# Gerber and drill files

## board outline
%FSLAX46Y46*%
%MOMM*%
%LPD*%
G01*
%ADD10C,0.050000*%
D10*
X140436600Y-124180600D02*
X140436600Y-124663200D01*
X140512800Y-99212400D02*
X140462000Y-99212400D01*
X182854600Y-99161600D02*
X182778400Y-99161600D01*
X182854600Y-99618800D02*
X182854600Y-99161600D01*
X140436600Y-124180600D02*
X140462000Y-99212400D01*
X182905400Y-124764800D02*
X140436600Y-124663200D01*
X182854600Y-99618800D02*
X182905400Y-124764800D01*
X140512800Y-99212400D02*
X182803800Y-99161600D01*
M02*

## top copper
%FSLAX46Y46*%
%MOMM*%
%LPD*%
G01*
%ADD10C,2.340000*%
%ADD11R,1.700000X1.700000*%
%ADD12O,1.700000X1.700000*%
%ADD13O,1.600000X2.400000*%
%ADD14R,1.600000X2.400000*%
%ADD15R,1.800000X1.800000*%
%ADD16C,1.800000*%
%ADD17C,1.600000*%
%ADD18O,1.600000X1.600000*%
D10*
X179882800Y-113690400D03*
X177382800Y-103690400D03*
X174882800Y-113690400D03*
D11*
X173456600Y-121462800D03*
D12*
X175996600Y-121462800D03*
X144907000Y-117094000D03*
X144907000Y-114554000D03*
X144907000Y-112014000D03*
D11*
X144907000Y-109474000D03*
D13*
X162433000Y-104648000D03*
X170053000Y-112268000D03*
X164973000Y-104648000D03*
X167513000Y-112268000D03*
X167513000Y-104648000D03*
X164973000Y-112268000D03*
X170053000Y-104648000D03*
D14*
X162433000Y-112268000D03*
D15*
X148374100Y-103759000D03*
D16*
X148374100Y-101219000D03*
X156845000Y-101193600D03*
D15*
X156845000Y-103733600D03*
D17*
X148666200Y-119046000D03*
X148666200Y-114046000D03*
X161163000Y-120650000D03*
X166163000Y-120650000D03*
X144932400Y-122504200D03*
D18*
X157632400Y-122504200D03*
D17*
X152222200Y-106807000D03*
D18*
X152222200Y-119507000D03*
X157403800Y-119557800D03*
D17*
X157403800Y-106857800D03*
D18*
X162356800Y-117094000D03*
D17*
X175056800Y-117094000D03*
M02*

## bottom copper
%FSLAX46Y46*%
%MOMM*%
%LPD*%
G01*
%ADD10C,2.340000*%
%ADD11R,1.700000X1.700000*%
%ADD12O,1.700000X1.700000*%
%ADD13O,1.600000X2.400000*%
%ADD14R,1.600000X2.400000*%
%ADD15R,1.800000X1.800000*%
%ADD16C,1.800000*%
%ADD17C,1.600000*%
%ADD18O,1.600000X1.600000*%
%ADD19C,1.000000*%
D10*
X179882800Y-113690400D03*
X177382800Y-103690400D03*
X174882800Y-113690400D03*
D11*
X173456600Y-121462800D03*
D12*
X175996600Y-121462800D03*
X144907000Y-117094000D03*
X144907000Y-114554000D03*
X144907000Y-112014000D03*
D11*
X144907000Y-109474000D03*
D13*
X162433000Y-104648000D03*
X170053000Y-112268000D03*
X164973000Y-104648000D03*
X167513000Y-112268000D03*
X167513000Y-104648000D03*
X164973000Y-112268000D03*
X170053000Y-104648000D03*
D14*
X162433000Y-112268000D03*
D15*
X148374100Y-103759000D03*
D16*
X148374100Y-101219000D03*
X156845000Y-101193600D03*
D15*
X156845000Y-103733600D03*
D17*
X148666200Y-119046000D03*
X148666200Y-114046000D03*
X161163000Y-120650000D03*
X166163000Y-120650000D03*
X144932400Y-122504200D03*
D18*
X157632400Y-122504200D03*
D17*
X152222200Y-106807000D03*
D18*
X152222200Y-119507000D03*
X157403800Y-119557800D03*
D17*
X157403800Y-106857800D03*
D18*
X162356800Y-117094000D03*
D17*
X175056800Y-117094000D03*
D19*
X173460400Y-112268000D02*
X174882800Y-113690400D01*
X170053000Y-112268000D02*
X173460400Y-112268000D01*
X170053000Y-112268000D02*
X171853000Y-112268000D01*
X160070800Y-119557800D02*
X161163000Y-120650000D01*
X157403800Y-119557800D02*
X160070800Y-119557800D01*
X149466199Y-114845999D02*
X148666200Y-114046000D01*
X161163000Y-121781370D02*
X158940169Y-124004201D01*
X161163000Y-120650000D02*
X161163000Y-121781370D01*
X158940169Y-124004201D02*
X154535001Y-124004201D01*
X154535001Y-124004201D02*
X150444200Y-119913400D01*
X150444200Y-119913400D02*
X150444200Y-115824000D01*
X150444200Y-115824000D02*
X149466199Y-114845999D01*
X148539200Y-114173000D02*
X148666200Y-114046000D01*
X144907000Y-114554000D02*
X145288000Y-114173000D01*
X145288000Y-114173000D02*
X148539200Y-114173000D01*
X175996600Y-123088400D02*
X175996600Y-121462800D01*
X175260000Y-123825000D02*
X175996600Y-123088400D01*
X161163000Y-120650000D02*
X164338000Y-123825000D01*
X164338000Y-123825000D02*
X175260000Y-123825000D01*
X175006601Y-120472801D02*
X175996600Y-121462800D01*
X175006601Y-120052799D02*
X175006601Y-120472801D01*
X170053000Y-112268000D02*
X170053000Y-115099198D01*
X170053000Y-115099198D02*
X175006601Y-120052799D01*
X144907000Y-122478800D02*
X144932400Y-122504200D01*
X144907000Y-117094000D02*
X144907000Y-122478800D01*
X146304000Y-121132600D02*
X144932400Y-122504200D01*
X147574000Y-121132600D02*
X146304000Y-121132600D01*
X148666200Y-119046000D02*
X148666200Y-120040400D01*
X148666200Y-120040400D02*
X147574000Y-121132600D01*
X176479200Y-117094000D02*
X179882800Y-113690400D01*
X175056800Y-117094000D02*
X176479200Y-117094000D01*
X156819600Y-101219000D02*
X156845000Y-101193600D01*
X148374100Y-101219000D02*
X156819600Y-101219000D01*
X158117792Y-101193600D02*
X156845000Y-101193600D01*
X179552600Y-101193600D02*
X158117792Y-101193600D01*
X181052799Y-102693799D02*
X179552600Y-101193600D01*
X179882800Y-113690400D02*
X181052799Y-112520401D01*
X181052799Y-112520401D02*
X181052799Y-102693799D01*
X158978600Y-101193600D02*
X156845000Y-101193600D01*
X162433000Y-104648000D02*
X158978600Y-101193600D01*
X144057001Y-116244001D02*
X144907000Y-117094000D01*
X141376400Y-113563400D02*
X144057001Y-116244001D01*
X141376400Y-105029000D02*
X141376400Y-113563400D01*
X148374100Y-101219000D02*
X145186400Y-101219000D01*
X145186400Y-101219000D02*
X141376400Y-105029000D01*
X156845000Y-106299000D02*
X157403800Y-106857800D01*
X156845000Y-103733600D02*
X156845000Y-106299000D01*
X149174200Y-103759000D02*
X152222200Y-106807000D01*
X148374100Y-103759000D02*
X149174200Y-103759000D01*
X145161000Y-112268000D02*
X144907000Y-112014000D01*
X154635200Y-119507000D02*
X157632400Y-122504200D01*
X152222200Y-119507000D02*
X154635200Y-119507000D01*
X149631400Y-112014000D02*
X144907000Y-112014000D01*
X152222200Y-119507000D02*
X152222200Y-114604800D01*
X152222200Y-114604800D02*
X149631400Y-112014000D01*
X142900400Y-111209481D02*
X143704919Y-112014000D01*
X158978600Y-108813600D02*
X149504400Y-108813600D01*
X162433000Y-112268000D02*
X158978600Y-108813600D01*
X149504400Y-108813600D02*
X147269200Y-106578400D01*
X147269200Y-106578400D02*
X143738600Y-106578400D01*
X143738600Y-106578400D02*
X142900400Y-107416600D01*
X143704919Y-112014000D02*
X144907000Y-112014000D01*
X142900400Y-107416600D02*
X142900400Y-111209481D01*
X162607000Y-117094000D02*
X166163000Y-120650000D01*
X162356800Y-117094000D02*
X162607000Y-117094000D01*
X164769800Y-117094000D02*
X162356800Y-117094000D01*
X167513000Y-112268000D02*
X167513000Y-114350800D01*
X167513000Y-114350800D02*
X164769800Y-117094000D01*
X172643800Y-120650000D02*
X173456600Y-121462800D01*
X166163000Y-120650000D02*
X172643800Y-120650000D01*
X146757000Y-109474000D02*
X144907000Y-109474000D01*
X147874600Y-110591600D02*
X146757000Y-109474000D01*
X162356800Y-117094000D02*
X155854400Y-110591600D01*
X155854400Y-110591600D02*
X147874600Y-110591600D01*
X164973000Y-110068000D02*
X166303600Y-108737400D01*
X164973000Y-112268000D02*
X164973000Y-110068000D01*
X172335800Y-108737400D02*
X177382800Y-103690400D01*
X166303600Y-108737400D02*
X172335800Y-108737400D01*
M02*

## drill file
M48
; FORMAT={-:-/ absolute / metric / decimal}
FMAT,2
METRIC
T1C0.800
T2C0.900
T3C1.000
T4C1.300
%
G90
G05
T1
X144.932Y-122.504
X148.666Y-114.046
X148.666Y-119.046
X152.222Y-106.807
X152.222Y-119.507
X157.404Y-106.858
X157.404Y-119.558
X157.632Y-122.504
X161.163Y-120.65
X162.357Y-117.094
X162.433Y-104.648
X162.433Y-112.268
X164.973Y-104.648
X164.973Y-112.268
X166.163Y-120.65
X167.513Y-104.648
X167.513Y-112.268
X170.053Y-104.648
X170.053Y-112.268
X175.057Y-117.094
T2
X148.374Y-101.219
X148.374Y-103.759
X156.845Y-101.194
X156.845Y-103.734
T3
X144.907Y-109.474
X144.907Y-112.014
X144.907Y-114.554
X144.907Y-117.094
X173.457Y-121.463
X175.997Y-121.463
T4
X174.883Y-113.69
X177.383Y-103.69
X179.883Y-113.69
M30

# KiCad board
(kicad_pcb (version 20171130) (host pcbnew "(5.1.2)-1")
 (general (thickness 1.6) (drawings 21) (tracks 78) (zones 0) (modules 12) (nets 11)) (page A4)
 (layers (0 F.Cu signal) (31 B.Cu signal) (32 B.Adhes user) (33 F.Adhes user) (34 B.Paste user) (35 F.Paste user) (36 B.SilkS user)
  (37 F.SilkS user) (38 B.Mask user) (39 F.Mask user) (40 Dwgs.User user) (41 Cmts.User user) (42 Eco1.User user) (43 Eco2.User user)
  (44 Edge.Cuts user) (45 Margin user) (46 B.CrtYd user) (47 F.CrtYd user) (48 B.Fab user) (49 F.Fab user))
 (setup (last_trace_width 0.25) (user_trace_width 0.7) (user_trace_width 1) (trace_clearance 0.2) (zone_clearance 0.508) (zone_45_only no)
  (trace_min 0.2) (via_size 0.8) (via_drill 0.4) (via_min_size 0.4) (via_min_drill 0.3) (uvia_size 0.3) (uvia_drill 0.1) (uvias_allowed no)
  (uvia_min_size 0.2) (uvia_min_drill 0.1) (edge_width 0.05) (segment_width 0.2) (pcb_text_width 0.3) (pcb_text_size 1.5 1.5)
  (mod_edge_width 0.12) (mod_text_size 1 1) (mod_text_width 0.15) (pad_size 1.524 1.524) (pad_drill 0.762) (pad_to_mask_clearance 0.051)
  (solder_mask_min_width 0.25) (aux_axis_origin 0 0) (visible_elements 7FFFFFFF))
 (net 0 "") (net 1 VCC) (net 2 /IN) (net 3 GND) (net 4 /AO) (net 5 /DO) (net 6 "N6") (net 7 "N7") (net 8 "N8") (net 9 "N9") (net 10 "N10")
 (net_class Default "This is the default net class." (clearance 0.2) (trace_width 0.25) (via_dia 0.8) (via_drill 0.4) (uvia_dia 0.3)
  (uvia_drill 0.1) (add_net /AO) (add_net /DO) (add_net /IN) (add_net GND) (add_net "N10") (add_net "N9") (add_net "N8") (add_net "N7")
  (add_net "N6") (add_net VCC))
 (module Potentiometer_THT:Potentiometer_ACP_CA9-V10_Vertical (layer F.Cu) (at 179.8828 113.6904 90)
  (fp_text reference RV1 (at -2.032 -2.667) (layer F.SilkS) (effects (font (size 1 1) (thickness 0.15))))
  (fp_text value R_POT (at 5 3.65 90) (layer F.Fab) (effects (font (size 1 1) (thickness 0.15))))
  (pad 1 thru_hole circle (at 0 0 90) (size 2.34 2.34) (drill 1.3) (layers *.Cu *.Mask) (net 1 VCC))
  (pad 2 thru_hole circle (at 10 -2.5 90) (size 2.34 2.34) (drill 1.3) (layers *.Cu *.Mask) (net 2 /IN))
  (pad 3 thru_hole circle (at 0 -5 90) (size 2.34 2.34) (drill 1.3) (layers *.Cu *.Mask) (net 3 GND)))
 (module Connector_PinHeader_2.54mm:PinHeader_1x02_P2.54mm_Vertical (layer F.Cu) (at 173.4566 121.4628 90)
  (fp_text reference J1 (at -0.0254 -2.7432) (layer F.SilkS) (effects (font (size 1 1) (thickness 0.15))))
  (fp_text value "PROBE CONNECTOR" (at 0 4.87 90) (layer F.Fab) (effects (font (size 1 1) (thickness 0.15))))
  (pad 1 thru_hole rect (at 0 0 90) (size 1.7 1.7) (drill 1) (layers *.Cu *.Mask) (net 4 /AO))
  (pad 2 thru_hole oval (at 0 2.54 90) (size 1.7 1.7) (drill 1) (layers *.Cu *.Mask) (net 3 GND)))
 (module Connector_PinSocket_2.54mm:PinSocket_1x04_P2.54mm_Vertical (layer F.Cu) (at 144.907 109.474)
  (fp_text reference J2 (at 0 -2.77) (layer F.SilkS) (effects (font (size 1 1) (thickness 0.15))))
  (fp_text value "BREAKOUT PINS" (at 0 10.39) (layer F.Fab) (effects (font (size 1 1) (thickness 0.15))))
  (pad 4 thru_hole oval (at 0 7.62) (size 1.7 1.7) (drill 1) (layers *.Cu *.Mask) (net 1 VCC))
  (pad 3 thru_hole oval (at 0 5.08) (size 1.7 1.7) (drill 1) (layers *.Cu *.Mask) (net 3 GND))
  (pad 2 thru_hole oval (at 0 2.54) (size 1.7 1.7) (drill 1) (layers *.Cu *.Mask) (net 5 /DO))
  (pad 1 thru_hole rect (at 0 0) (size 1.7 1.7) (drill 1) (layers *.Cu *.Mask) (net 4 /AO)))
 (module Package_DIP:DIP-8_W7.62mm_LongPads (layer F.Cu) (at 162.433 112.268 90)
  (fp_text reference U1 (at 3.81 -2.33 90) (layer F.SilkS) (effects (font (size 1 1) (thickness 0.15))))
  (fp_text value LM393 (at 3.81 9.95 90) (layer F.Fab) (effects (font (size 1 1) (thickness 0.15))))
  (pad 8 thru_hole oval (at 7.62 0 90) (size 2.4 1.6) (drill 0.8) (layers *.Cu *.Mask) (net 1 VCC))
  (pad 4 thru_hole oval (at 0 7.62 90) (size 2.4 1.6) (drill 0.8) (layers *.Cu *.Mask) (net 3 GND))
  (pad 7 thru_hole oval (at 7.62 2.54 90) (size 2.4 1.6) (drill 0.8) (layers *.Cu *.Mask) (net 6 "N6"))
  (pad 3 thru_hole oval (at 0 5.08 90) (size 2.4 1.6) (drill 0.8) (layers *.Cu *.Mask) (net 4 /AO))
  (pad 6 thru_hole oval (at 7.62 5.08 90) (size 2.4 1.6) (drill 0.8) (layers *.Cu *.Mask) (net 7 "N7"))
  (pad 2 thru_hole oval (at 0 2.54 90) (size 2.4 1.6) (drill 0.8) (layers *.Cu *.Mask) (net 2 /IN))
  (pad 5 thru_hole oval (at 7.62 7.62 90) (size 2.4 1.6) (drill 0.8) (layers *.Cu *.Mask) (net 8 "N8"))
  (pad 1 thru_hole rect (at 0 0 90) (size 2.4 1.6) (drill 0.8) (layers *.Cu *.Mask) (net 5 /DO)))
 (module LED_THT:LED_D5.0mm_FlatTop (layer F.Cu) (at 148.3741 103.759 90)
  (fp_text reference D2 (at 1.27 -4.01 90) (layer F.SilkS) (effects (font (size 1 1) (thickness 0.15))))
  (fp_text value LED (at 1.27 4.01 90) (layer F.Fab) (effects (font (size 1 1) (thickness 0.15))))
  (pad 1 thru_hole rect (at 0 0 90) (size 1.8 1.8) (drill 0.9) (layers *.Cu *.Mask) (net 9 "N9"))
  (pad 2 thru_hole circle (at 2.54 0 90) (size 1.8 1.8) (drill 0.9) (layers *.Cu *.Mask) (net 1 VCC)))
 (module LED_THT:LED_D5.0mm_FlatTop (layer F.Cu) (at 156.845 103.7336 90)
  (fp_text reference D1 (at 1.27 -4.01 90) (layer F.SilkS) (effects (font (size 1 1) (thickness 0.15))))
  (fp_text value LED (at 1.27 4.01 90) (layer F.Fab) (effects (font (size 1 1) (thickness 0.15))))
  (pad 2 thru_hole circle (at 2.54 0 90) (size 1.8 1.8) (drill 0.9) (layers *.Cu *.Mask) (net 1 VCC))
  (pad 1 thru_hole rect (at 0 0 90) (size 1.8 1.8) (drill 0.9) (layers *.Cu *.Mask) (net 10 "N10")))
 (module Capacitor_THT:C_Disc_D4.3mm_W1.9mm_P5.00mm (layer F.Cu) (at 148.6662 114.046 270)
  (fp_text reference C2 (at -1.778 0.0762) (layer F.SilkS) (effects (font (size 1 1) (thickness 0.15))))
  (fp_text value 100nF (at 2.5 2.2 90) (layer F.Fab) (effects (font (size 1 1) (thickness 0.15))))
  (pad 2 thru_hole circle (at 5 0 270) (size 1.6 1.6) (drill 0.8) (layers *.Cu *.Mask) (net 1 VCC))
  (pad 1 thru_hole circle (at 0 0 270) (size 1.6 1.6) (drill 0.8) (layers *.Cu *.Mask) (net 3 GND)))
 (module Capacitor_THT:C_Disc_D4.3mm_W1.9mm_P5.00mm (layer F.Cu) (at 161.163 120.65)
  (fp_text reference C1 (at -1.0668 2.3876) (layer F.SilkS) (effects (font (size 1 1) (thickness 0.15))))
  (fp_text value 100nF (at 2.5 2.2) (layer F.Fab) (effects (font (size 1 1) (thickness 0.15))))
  (pad 1 thru_hole circle (at 0 0) (size 1.6 1.6) (drill 0.8) (layers *.Cu *.Mask) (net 3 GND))
  (pad 2 thru_hole circle (at 5 0) (size 1.6 1.6) (drill 0.8) (layers *.Cu *.Mask) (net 4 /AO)))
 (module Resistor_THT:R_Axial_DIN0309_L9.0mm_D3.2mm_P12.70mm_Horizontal (layer F.Cu) (at 144.9324 122.5042)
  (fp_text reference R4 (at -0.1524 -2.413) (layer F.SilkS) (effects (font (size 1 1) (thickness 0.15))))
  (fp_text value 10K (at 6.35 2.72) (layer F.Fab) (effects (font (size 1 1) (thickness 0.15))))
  (pad 1 thru_hole circle (at 0 0) (size 1.6 1.6) (drill 0.8) (layers *.Cu *.Mask) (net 1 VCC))
  (pad 2 thru_hole oval (at 12.7 0) (size 1.6 1.6) (drill 0.8) (layers *.Cu *.Mask) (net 5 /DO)))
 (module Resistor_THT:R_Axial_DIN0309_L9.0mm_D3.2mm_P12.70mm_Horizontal (layer F.Cu) (at 152.2222 106.807 270)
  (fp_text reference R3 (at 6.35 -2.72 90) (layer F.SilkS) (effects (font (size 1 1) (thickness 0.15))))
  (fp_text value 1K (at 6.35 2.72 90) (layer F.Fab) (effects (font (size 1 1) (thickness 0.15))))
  (pad 1 thru_hole circle (at 0 0 270) (size 1.6 1.6) (drill 0.8) (layers *.Cu *.Mask) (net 9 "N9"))
  (pad 2 thru_hole oval (at 12.7 0 270) (size 1.6 1.6) (drill 0.8) (layers *.Cu *.Mask) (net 5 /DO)))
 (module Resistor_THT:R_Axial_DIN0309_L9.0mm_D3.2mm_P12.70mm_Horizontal (layer F.Cu) (at 157.4038 106.8578 270)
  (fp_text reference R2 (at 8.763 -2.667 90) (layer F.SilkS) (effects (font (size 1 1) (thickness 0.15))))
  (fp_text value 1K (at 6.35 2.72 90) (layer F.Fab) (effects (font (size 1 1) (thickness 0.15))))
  (pad 2 thru_hole oval (at 12.7 0 270) (size 1.6 1.6) (drill 0.8) (layers *.Cu *.Mask) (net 3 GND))
  (pad 1 thru_hole circle (at 0 0 270) (size 1.6 1.6) (drill 0.8) (layers *.Cu *.Mask) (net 10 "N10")))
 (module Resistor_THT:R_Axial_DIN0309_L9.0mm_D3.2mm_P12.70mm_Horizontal (layer F.Cu) (at 175.0568 117.094 180)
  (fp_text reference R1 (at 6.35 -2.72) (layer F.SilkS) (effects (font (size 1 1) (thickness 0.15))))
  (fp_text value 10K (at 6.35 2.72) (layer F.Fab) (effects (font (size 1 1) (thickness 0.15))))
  (pad 2 thru_hole oval (at 12.7 0 180) (size 1.6 1.6) (drill 0.8) (layers *.Cu *.Mask) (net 4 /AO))
  (pad 1 thru_hole circle (at 0 0 180) (size 1.6 1.6) (drill 0.8) (layers *.Cu *.Mask) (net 1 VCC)))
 (gr_line (start 140.4366 124.1806) (end 140.4366 124.6632) (layer Edge.Cuts) (width 0.05))
 (gr_line (start 140.5128 99.2124) (end 140.462 99.2124) (layer Edge.Cuts) (width 0.05))
 (gr_line (start 182.8546 99.1616) (end 182.7784 99.1616) (layer Edge.Cuts) (width 0.05))
 (gr_line (start 182.8546 99.6188) (end 182.8546 99.1616) (layer Edge.Cuts) (width 0.05))
 (gr_line (start 140.4366 124.1806) (end 140.462 99.2124) (layer Edge.Cuts) (width 0.05))
 (gr_line (start 182.9054 124.7648) (end 140.4366 124.6632) (layer Edge.Cuts) (width 0.05))
 (gr_line (start 182.8546 99.6188) (end 182.9054 124.7648) (layer Edge.Cuts) (width 0.05))
 (gr_line (start 140.5128 99.2124) (end 182.8038 99.1616) (layer Edge.Cuts) (width 0.05))
 (segment (start 173.4604 112.268) (end 174.8828 113.6904) (width 1) (layer B.Cu) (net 3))
 (segment (start 170.053 112.268) (end 173.4604 112.268) (width 1) (layer B.Cu) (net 3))
 (segment (start 170.053 112.268) (end 171.853 112.268) (width 1) (layer B.Cu) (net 3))
 (segment (start 160.0708 119.5578) (end 161.163 120.65) (width 1) (layer B.Cu) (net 3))
 (segment (start 157.4038 119.5578) (end 160.0708 119.5578) (width 1) (layer B.Cu) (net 3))
 (segment (start 149.466199 114.845999) (end 148.6662 114.046) (width 1) (layer B.Cu) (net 3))
 (segment (start 161.163 121.78137) (end 158.940169 124.004201) (width 1) (layer B.Cu) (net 3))
 (segment (start 161.163 120.65) (end 161.163 121.78137) (width 1) (layer B.Cu) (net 3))
 (segment (start 158.940169 124.004201) (end 154.535001 124.004201) (width 1) (layer B.Cu) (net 3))
 (segment (start 154.535001 124.004201) (end 150.4442 119.9134) (width 1) (layer B.Cu) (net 3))
 (segment (start 150.4442 119.9134) (end 150.4442 115.824) (width 1) (layer B.Cu) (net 3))
 (segment (start 150.4442 115.824) (end 149.466199 114.845999) (width 1) (layer B.Cu) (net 3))
 (segment (start 148.5392 114.173) (end 148.6662 114.046) (width 1) (layer B.Cu) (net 3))
 (segment (start 144.907 114.554) (end 145.288 114.173) (width 1) (layer B.Cu) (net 3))
 (segment (start 145.288 114.173) (end 148.5392 114.173) (width 1) (layer B.Cu) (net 3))
 (segment (start 175.9966 123.0884) (end 175.9966 121.4628) (width 1) (layer B.Cu) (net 3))
 (segment (start 175.26 123.825) (end 175.9966 123.0884) (width 1) (layer B.Cu) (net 3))
 (segment (start 161.163 120.65) (end 164.338 123.825) (width 1) (layer B.Cu) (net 3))
 (segment (start 164.338 123.825) (end 175.26 123.825) (width 1) (layer B.Cu) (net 3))
 (segment (start 175.006601 120.472801) (end 175.9966 121.4628) (width 1) (layer B.Cu) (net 3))
 (segment (start 175.006601 120.052799) (end 175.006601 120.472801) (width 1) (layer B.Cu) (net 3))
 (segment (start 170.053 112.268) (end 170.053 115.099198) (width 1) (layer B.Cu) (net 3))
 (segment (start 170.053 115.099198) (end 175.006601 120.052799) (width 1) (layer B.Cu) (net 3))
 (segment (start 144.907 122.4788) (end 144.9324 122.5042) (width 1) (layer B.Cu) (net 1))
 (segment (start 144.907 117.094) (end 144.907 122.4788) (width 1) (layer B.Cu) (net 1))
 (segment (start 146.304 121.1326) (end 144.9324 122.5042) (width 1) (layer B.Cu) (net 1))
 (segment (start 147.574 121.1326) (end 146.304 121.1326) (width 1) (layer B.Cu) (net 1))
 (segment (start 148.6662 119.046) (end 148.6662 120.0404) (width 1) (layer B.Cu) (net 1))
 (segment (start 148.6662 120.0404) (end 147.574 121.1326) (width 1) (layer B.Cu) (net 1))
 (segment (start 176.4792 117.094) (end 179.8828 113.6904) (width 1) (layer B.Cu) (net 1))
 (segment (start 175.0568 117.094) (end 176.4792 117.094) (width 1) (layer B.Cu) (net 1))
 (segment (start 156.8196 101.219) (end 156.845 101.1936) (width 1) (layer B.Cu) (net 1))
 (segment (start 148.3741 101.219) (end 156.8196 101.219) (width 1) (layer B.Cu) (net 1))
 (segment (start 158.117792 101.1936) (end 156.845 101.1936) (width 1) (layer B.Cu) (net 1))
 (segment (start 179.5526 101.1936) (end 158.117792 101.1936) (width 1) (layer B.Cu) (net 1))
 (segment (start 181.052799 102.693799) (end 179.5526 101.1936) (width 1) (layer B.Cu) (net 1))
 (segment (start 179.8828 113.6904) (end 181.052799 112.520401) (width 1) (layer B.Cu) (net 1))
 (segment (start 181.052799 112.520401) (end 181.052799 102.693799) (width 1) (layer B.Cu) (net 1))
 (segment (start 158.9786 101.1936) (end 156.845 101.1936) (width 1) (layer B.Cu) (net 1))
 (segment (start 162.433 104.648) (end 158.9786 101.1936) (width 1) (layer B.Cu) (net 1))
 (segment (start 144.057001 116.244001) (end 144.907 117.094) (width 1) (layer B.Cu) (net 1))
 (segment (start 141.3764 113.5634) (end 144.057001 116.244001) (width 1) (layer B.Cu) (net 1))
 (segment (start 141.3764 105.029) (end 141.3764 113.5634) (width 1) (layer B.Cu) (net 1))
 (segment (start 148.3741 101.219) (end 145.1864 101.219) (width 1) (layer B.Cu) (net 1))
 (segment (start 145.1864 101.219) (end 141.3764 105.029) (width 1) (layer B.Cu) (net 1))
 (segment (start 156.845 106.299) (end 157.4038 106.8578) (width 1) (layer B.Cu) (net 10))
 (segment (start 156.845 103.7336) (end 156.845 106.299) (width 1) (layer B.Cu) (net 10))
 (segment (start 149.1742 103.759) (end 152.2222 106.807) (width 1) (layer B.Cu) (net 9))
 (segment (start 148.3741 103.759) (end 149.1742 103.759) (width 1) (layer B.Cu) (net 9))
 (segment (start 145.161 112.268) (end 144.907 112.014) (width 1) (layer B.Cu) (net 5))
 (segment (start 154.6352 119.507) (end 157.6324 122.5042) (width 1) (layer B.Cu) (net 5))
 (segment (start 152.2222 119.507) (end 154.6352 119.507) (width 1) (layer B.Cu) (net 5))
 (segment (start 149.6314 112.014) (end 144.907 112.014) (width 1) (layer B.Cu) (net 5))
 (segment (start 152.2222 119.507) (end 152.2222 114.6048) (width 1) (layer B.Cu) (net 5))
 (segment (start 152.2222 114.6048) (end 149.6314 112.014) (width 1) (layer B.Cu) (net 5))
 (segment (start 142.9004 111.209481) (end 143.704919 112.014) (width 1) (layer B.Cu) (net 5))
 (segment (start 158.9786 108.8136) (end 149.5044 108.8136) (width 1) (layer B.Cu) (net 5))
 (segment (start 162.433 112.268) (end 158.9786 108.8136) (width 1) (layer B.Cu) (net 5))
 (segment (start 149.5044 108.8136) (end 147.2692 106.5784) (width 1) (layer B.Cu) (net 5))
 (segment (start 147.2692 106.5784) (end 143.7386 106.5784) (width 1) (layer B.Cu) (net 5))
 (segment (start 143.7386 106.5784) (end 142.9004 107.4166) (width 1) (layer B.Cu) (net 5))
 (segment (start 143.704919 112.014) (end 144.907 112.014) (width 1) (layer B.Cu) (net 5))
 (segment (start 142.9004 107.4166) (end 142.9004 111.209481) (width 1) (layer B.Cu) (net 5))
 (segment (start 162.607 117.094) (end 166.163 120.65) (width 1) (layer B.Cu) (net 4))
 (segment (start 162.3568 117.094) (end 162.607 117.094) (width 1) (layer B.Cu) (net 4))
 (segment (start 164.7698 117.094) (end 162.3568 117.094) (width 1) (layer B.Cu) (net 4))
 (segment (start 167.513 112.268) (end 167.513 114.3508) (width 1) (layer B.Cu) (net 4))
 (segment (start 167.513 114.3508) (end 164.7698 117.094) (width 1) (layer B.Cu) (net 4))
 (segment (start 172.6438 120.65) (end 173.4566 121.4628) (width 1) (layer B.Cu) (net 4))
 (segment (start 166.163 120.65) (end 172.6438 120.65) (width 1) (layer B.Cu) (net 4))
 (segment (start 146.757 109.474) (end 144.907 109.474) (width 1) (layer B.Cu) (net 4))
 (segment (start 147.8746 110.5916) (end 146.757 109.474) (width 1) (layer B.Cu) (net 4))
 (segment (start 162.3568 117.094) (end 155.8544 110.5916) (width 1) (layer B.Cu) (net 4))
 (segment (start 155.8544 110.5916) (end 147.8746 110.5916) (width 1) (layer B.Cu) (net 4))
 (segment (start 164.973 110.068) (end 166.3036 108.7374) (width 1) (layer B.Cu) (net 2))
 (segment (start 164.973 112.268) (end 164.973 110.068) (width 1) (layer B.Cu) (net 2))
 (segment (start 172.3358 108.7374) (end 177.3828 103.6904) (width 1) (layer B.Cu) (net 2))
 (segment (start 166.3036 108.7374) (end 172.3358 108.7374) (width 1) (layer B.Cu) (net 2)))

